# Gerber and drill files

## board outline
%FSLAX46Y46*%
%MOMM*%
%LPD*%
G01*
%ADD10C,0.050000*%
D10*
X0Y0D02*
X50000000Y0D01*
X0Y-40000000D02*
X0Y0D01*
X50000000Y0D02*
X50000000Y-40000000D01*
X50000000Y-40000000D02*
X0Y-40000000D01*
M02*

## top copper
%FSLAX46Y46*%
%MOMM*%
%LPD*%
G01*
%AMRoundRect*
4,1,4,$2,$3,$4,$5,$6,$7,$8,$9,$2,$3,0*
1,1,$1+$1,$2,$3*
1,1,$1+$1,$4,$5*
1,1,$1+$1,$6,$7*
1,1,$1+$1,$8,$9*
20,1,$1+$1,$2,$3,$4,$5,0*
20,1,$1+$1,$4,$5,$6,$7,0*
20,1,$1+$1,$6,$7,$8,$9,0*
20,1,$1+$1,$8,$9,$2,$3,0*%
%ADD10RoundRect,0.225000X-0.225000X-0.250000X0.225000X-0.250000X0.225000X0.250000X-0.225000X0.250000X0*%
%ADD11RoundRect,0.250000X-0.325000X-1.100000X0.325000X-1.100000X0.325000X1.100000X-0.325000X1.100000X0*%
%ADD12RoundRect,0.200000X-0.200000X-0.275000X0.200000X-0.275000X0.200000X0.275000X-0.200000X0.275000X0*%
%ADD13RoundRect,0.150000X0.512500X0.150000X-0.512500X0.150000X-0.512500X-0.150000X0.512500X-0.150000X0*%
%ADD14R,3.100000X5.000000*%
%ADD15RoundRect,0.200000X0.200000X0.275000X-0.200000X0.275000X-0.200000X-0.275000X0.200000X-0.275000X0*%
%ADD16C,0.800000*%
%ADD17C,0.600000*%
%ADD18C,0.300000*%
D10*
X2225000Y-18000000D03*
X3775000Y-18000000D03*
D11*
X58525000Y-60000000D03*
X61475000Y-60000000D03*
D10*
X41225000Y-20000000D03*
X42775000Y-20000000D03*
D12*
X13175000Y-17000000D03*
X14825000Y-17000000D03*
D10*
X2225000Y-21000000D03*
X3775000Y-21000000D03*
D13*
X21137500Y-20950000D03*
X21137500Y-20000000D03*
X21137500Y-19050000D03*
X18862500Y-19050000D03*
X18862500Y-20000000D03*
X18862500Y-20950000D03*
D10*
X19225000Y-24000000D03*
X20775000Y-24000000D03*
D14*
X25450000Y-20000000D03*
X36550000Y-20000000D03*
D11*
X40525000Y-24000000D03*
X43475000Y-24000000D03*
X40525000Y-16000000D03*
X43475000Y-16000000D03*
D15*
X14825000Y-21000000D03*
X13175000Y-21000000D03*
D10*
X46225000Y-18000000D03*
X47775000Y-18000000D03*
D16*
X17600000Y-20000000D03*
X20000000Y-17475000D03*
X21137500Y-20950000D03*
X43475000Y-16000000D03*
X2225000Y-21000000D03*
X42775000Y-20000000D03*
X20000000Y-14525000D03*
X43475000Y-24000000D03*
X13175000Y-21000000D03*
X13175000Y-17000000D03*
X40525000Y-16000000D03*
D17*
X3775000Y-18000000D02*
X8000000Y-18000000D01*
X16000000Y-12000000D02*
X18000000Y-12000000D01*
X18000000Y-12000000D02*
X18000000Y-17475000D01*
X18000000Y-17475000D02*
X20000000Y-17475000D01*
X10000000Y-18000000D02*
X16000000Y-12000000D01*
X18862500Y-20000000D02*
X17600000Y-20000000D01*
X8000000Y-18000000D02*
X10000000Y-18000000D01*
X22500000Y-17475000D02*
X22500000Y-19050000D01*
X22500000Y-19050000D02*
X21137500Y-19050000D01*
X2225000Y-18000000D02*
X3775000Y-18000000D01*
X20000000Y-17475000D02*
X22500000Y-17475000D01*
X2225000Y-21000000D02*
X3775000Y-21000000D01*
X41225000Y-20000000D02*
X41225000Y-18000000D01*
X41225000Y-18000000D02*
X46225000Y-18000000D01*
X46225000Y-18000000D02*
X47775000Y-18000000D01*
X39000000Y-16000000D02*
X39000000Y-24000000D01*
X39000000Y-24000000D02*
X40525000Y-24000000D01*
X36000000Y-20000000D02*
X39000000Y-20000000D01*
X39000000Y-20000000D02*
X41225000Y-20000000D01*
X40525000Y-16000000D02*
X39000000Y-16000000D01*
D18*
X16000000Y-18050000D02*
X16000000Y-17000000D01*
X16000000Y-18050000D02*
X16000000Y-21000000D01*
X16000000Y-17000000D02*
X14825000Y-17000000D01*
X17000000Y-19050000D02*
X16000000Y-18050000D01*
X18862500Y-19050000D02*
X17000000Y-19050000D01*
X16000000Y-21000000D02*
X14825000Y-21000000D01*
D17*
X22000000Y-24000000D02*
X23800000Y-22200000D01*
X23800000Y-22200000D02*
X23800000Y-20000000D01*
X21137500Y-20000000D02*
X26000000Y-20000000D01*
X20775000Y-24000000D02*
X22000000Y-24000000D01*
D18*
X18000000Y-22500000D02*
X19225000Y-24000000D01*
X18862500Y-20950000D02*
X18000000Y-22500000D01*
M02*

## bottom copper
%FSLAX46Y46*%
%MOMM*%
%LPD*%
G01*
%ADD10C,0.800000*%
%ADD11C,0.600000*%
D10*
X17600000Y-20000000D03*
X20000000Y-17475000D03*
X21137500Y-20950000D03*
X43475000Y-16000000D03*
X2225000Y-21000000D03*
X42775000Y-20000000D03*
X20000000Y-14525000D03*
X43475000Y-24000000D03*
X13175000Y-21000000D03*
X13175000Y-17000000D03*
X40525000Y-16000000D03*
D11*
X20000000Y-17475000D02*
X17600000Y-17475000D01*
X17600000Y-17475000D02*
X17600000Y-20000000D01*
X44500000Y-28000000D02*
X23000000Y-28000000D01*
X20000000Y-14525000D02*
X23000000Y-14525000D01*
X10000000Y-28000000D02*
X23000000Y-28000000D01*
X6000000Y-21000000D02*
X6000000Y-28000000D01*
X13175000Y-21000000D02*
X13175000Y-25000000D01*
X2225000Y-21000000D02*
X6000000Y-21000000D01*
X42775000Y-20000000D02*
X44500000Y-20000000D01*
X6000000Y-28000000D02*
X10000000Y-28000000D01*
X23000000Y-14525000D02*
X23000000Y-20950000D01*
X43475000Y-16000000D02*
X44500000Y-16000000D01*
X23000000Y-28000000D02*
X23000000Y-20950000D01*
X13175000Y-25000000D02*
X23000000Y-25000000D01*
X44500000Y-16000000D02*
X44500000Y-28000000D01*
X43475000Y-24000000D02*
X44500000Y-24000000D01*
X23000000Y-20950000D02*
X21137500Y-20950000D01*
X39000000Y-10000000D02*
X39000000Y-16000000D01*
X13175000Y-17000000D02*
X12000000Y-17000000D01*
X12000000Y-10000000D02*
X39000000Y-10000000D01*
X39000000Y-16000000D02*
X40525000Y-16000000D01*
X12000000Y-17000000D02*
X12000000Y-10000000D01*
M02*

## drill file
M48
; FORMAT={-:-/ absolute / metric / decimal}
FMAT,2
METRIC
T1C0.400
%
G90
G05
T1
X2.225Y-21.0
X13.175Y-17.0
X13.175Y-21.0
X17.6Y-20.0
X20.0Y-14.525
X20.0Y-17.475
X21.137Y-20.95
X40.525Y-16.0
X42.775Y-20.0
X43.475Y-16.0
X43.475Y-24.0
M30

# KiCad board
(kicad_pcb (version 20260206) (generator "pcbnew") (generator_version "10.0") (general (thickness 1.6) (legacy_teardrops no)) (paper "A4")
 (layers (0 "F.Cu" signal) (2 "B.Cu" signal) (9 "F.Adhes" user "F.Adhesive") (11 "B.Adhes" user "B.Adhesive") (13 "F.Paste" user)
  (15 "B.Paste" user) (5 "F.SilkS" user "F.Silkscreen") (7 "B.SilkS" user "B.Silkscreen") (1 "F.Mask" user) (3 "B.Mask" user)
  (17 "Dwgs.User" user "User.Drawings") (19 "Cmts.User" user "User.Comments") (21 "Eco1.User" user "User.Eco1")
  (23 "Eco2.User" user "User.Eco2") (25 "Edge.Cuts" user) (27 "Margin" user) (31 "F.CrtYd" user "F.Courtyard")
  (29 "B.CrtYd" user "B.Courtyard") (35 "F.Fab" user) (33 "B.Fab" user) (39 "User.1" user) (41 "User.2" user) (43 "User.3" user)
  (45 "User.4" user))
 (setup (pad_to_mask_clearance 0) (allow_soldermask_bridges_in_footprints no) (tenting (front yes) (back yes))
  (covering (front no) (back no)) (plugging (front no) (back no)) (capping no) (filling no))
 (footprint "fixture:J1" (layer "F.Cu") (at 3 18)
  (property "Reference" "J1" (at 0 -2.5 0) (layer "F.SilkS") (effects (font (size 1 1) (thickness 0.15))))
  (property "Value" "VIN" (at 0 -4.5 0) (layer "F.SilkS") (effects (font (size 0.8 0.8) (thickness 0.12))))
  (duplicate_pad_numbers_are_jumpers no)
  (pad "1" smd roundrect (at -0.775 0) (size 0.9 0.95) (layers "F.Cu" "F.Mask" "F.Paste") (roundrect_rratio 0.25) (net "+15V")
   (thermal_bridge_angle 45))
  (pad "2" smd roundrect (at 0.775 0) (size 0.9 0.95) (layers "F.Cu" "F.Mask" "F.Paste") (roundrect_rratio 0.25) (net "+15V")
   (thermal_bridge_angle 45)))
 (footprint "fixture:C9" (layer "F.Cu") (at 60 60)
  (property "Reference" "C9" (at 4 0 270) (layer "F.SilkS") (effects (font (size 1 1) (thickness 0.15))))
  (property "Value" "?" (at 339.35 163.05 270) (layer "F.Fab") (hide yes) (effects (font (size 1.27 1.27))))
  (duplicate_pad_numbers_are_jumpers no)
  (pad "1" smd roundrect (at -1.475 0) (size 1.15 2.7) (layers "F.Cu" "F.Mask" "F.Paste") (roundrect_rratio 0.217391) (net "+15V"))
  (pad "2" smd roundrect (at 1.475 0) (size 1.15 2.7) (layers "F.Cu" "F.Mask" "F.Paste") (roundrect_rratio 0.217391) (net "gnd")))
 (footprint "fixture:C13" (layer "F.Cu") (at 42 20)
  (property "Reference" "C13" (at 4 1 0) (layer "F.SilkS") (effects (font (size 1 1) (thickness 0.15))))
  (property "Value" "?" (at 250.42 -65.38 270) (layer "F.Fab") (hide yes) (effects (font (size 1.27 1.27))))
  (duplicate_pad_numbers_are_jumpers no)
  (pad "1" smd roundrect (at -0.775 0) (size 0.9 0.95) (layers "F.Cu" "F.Mask" "F.Paste") (roundrect_rratio 0.25) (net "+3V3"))
  (pad "2" smd roundrect (at 0.775 0) (size 0.9 0.95) (layers "F.Cu" "F.Mask" "F.Paste") (roundrect_rratio 0.25) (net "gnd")))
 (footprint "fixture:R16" (layer "F.Cu") (at 14 17)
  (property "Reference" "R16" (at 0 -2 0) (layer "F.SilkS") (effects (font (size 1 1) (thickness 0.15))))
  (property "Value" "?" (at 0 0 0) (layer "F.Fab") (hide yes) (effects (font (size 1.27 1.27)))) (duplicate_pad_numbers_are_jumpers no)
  (pad "1" smd roundrect (at -0.825 0) (size 0.8 0.95) (layers "F.Cu" "F.Mask" "F.Paste") (roundrect_rratio 0.25) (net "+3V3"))
  (pad "2" smd roundrect (at 0.825 0) (size 0.8 0.95) (layers "F.Cu" "F.Mask" "F.Paste") (roundrect_rratio 0.25) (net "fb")))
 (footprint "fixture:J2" (layer "F.Cu") (at 3 21)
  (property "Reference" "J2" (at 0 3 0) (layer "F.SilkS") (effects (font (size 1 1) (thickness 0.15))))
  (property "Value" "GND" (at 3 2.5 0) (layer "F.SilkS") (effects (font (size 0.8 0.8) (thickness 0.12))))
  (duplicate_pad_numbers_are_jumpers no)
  (pad "1" smd roundrect (at -0.775 0) (size 0.9 0.95) (layers "F.Cu" "F.Mask" "F.Paste") (roundrect_rratio 0.25) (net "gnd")
   (thermal_bridge_angle 45))
  (pad "2" smd roundrect (at 0.775 0) (size 0.9 0.95) (layers "F.Cu" "F.Mask" "F.Paste") (roundrect_rratio 0.25) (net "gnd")
   (thermal_bridge_angle 45)))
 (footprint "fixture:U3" (layer "F.Cu") (at 20 20 180)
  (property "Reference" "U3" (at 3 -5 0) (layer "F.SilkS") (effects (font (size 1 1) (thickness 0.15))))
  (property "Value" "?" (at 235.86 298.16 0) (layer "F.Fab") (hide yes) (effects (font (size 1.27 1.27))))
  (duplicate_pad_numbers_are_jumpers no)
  (pad "1" smd roundrect (at -1.1375 -0.95 180) (size 1.325 0.6) (layers "F.Cu" "F.Mask" "F.Paste") (roundrect_rratio 0.25) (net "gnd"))
  (pad "2" smd roundrect (at -1.1375 0 180) (size 1.325 0.6) (layers "F.Cu" "F.Mask" "F.Paste") (roundrect_rratio 0.25) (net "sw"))
  (pad "3" smd roundrect (at -1.1375 0.95 180) (size 1.325 0.6) (layers "F.Cu" "F.Mask" "F.Paste") (roundrect_rratio 0.25) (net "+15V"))
  (pad "4" smd roundrect (at 1.1375 0.95 180) (size 1.325 0.6) (layers "F.Cu" "F.Mask" "F.Paste") (roundrect_rratio 0.25) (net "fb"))
  (pad "5" smd roundrect (at 1.1375 0 180) (size 1.325 0.6) (layers "F.Cu" "F.Mask" "F.Paste") (roundrect_rratio 0.25) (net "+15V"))
  (pad "6" smd roundrect (at 1.1375 -0.95 180) (size 1.325 0.6) (layers "F.Cu" "F.Mask" "F.Paste") (roundrect_rratio 0.25) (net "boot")))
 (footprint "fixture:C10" (layer "F.Cu") (at 20 24)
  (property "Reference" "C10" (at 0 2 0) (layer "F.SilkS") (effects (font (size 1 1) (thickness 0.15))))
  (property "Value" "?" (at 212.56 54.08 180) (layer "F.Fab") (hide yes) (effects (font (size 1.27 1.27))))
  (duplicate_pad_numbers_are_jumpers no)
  (pad "1" smd roundrect (at -0.775 0) (size 0.9 0.95) (layers "F.Cu" "F.Mask" "F.Paste") (roundrect_rratio 0.25) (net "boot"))
  (pad "2" smd roundrect (at 0.775 0) (size 0.9 0.95) (layers "F.Cu" "F.Mask" "F.Paste") (roundrect_rratio 0.25) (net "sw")))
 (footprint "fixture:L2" (layer "F.Cu") (at 31 20)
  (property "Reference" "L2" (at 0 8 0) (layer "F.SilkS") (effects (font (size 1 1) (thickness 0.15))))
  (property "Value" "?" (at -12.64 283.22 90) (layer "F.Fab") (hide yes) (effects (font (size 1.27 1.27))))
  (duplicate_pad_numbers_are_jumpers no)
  (pad "1" smd rect (at -5.55 0) (size 3.1 5) (layers "F.Cu" "F.Mask" "F.Paste") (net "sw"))
  (pad "2" smd rect (at 5.55 0) (size 3.1 5) (layers "F.Cu" "F.Mask" "F.Paste") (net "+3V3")))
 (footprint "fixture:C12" (layer "F.Cu") (at 42 24)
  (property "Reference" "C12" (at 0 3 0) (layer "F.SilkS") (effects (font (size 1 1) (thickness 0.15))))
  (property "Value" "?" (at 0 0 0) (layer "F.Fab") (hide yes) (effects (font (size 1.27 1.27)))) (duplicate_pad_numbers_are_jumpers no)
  (pad "1" smd roundrect (at -1.475 0) (size 1.15 2.7) (layers "F.Cu" "F.Mask" "F.Paste") (roundrect_rratio 0.217391) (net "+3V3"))
  (pad "2" smd roundrect (at 1.475 0) (size 1.15 2.7) (layers "F.Cu" "F.Mask" "F.Paste") (roundrect_rratio 0.217391) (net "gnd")))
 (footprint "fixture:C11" (layer "F.Cu") (at 42 16)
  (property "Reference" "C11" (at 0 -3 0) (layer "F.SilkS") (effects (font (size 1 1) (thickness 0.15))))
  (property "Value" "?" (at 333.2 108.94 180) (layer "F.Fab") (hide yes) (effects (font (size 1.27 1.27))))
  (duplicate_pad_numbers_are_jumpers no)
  (pad "1" smd roundrect (at -1.475 0) (size 1.15 2.7) (layers "F.Cu" "F.Mask" "F.Paste") (roundrect_rratio 0.217391) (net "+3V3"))
  (pad "2" smd roundrect (at 1.475 0) (size 1.15 2.7) (layers "F.Cu" "F.Mask" "F.Paste") (roundrect_rratio 0.217391) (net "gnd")))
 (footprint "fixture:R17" (layer "F.Cu") (at 14 21 180)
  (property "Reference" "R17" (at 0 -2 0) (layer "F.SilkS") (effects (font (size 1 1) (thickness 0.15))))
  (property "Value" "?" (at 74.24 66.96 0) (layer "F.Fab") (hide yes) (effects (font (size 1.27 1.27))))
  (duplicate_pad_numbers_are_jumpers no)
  (pad "1" smd roundrect (at -0.825 0 180) (size 0.8 0.95) (layers "F.Cu" "F.Mask" "F.Paste") (roundrect_rratio 0.25) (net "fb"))
  (pad "2" smd roundrect (at 0.825 0 180) (size 0.8 0.95) (layers "F.Cu" "F.Mask" "F.Paste") (roundrect_rratio 0.25) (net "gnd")))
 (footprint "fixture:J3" (layer "F.Cu") (at 47 18)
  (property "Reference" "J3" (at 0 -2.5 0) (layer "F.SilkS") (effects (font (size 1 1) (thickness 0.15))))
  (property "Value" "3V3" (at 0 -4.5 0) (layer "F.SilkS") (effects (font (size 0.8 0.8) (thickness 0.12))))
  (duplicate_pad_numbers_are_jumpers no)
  (pad "1" smd roundrect (at -0.775 0) (size 0.9 0.95) (layers "F.Cu" "F.Mask" "F.Paste") (roundrect_rratio 0.25) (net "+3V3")
   (thermal_bridge_angle 45))
  (pad "2" smd roundrect (at 0.775 0) (size 0.9 0.95) (layers "F.Cu" "F.Mask" "F.Paste") (roundrect_rratio 0.25) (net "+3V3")
   (thermal_bridge_angle 45)))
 (gr_line (start 0 0) (end 50 0) (stroke (width 0.05) (type default)) (layer "Edge.Cuts"))
 (gr_line (start 0 40) (end 0 0) (stroke (width 0.05) (type default)) (layer "Edge.Cuts"))
 (gr_line (start 50 0) (end 50 40) (stroke (width 0.05) (type default)) (layer "Edge.Cuts"))
 (gr_line (start 50 40) (end 0 40) (stroke (width 0.05) (type default)) (layer "Edge.Cuts"))
 (segment (start 3.775 18) (end 8 18) (width 0.6) (layer "F.Cu") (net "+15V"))
 (segment (start 16 12) (end 18 12) (width 0.6) (layer "F.Cu") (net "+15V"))
 (segment (start 18 12) (end 18 17.475) (width 0.6) (layer "F.Cu") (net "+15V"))
 (segment (start 18 17.475) (end 20 17.475) (width 0.6) (layer "F.Cu") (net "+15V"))
 (segment (start 10 18) (end 16 12) (width 0.6) (layer "F.Cu") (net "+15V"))
 (segment (start 18.8625 20) (end 17.6 20) (width 0.6) (layer "F.Cu") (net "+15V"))
 (segment (start 8 18) (end 10 18) (width 0.6) (layer "F.Cu") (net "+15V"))
 (segment (start 22.5 17.475) (end 22.5 19.05) (width 0.6) (layer "F.Cu") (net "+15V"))
 (segment (start 22.5 19.05) (end 21.1375 19.05) (width 0.6) (layer "F.Cu") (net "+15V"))
 (segment (start 2.225 18) (end 3.775 18) (width 0.6) (layer "F.Cu") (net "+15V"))
 (segment (start 20 17.475) (end 22.5 17.475) (width 0.6) (layer "F.Cu") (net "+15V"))
 (via (at 17.6 20) (size 0.8) (drill 0.4) (layers "F.Cu" "B.Cu") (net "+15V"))
 (via (at 20 17.475) (size 0.8) (drill 0.4) (layers "F.Cu" "B.Cu") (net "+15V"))
 (segment (start 20 17.475) (end 17.6 17.475) (width 0.6) (layer "B.Cu") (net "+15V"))
 (segment (start 17.6 17.475) (end 17.6 20) (width 0.6) (layer "B.Cu") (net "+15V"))
 (segment (start 2.225 21) (end 3.775 21) (width 0.6) (layer "F.Cu") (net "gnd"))
 (via (at 21.1375 20.95) (size 0.8) (drill 0.4) (layers "F.Cu" "B.Cu") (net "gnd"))
 (via (at 43.475 16) (size 0.8) (drill 0.4) (layers "F.Cu" "B.Cu") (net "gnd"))
 (via (at 2.225 21) (size 0.8) (drill 0.4) (layers "F.Cu" "B.Cu") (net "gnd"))
 (via (at 42.775 20) (size 0.8) (drill 0.4) (layers "F.Cu" "B.Cu") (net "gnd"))
 (via (at 20 14.525) (size 0.8) (drill 0.4) (layers "F.Cu" "B.Cu") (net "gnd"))
 (via (at 43.475 24) (size 0.8) (drill 0.4) (layers "F.Cu" "B.Cu") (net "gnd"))
 (via (at 13.175 21) (size 0.8) (drill 0.4) (layers "F.Cu" "B.Cu") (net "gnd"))
 (segment (start 44.5 28) (end 23 28) (width 0.6) (layer "B.Cu") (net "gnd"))
 (segment (start 20 14.525) (end 23 14.525) (width 0.6) (layer "B.Cu") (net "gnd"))
 (segment (start 10 28) (end 23 28) (width 0.6) (layer "B.Cu") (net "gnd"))
 (segment (start 6 21) (end 6 28) (width 0.6) (layer "B.Cu") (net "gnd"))
 (segment (start 13.175 21) (end 13.175 25) (width 0.6) (layer "B.Cu") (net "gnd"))
 (segment (start 2.225 21) (end 6 21) (width 0.6) (layer "B.Cu") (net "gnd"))
 (segment (start 42.775 20) (end 44.5 20) (width 0.6) (layer "B.Cu") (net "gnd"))
 (segment (start 6 28) (end 10 28) (width 0.6) (layer "B.Cu") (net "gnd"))
 (segment (start 23 14.525) (end 23 20.95) (width 0.6) (layer "B.Cu") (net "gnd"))
 (segment (start 43.475 16) (end 44.5 16) (width 0.6) (layer "B.Cu") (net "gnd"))
 (segment (start 23 28) (end 23 20.95) (width 0.6) (layer "B.Cu") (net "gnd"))
 (segment (start 13.175 25) (end 23 25) (width 0.6) (layer "B.Cu") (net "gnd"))
 (segment (start 44.5 16) (end 44.5 28) (width 0.6) (layer "B.Cu") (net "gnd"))
 (segment (start 43.475 24) (end 44.5 24) (width 0.6) (layer "B.Cu") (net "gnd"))
 (segment (start 23 20.95) (end 21.1375 20.95) (width 0.6) (layer "B.Cu") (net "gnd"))
 (segment (start 41.225 20) (end 41.225 18) (width 0.6) (layer "F.Cu") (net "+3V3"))
 (segment (start 41.225 18) (end 46.225 18) (width 0.6) (layer "F.Cu") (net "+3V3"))
 (segment (start 46.225 18) (end 47.775 18) (width 0.6) (layer "F.Cu") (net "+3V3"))
 (segment (start 39 16) (end 39 24) (width 0.6) (layer "F.Cu") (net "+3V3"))
 (segment (start 39 24) (end 40.525 24) (width 0.6) (layer "F.Cu") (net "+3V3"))
 (segment (start 36 20) (end 39 20) (width 0.6) (layer "F.Cu") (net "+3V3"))
 (segment (start 39 20) (end 41.225 20) (width 0.6) (layer "F.Cu") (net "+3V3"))
 (segment (start 40.525 16) (end 39 16) (width 0.6) (layer "F.Cu") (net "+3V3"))
 (via (at 13.175 17) (size 0.8) (drill 0.4) (layers "F.Cu" "B.Cu") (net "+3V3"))
 (via (at 40.525 16) (size 0.8) (drill 0.4) (layers "F.Cu" "B.Cu") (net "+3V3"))
 (segment (start 39 10) (end 39 16) (width 0.6) (layer "B.Cu") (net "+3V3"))
 (segment (start 13.175 17) (end 12 17) (width 0.6) (layer "B.Cu") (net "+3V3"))
 (segment (start 12 10) (end 39 10) (width 0.6) (layer "B.Cu") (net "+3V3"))
 (segment (start 39 16) (end 40.525 16) (width 0.6) (layer "B.Cu") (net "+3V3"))
 (segment (start 12 17) (end 12 10) (width 0.6) (layer "B.Cu") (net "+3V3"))
 (segment (start 16 18.05) (end 16 17) (width 0.3) (layer "F.Cu") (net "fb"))
 (segment (start 16 18.05) (end 16 21) (width 0.3) (layer "F.Cu") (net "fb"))
 (segment (start 16 17) (end 14.825 17) (width 0.3) (layer "F.Cu") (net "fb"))
 (segment (start 17 19.05) (end 16 18.05) (width 0.3) (layer "F.Cu") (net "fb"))
 (segment (start 18.8625 19.05) (end 17 19.05) (width 0.3) (layer "F.Cu") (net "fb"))
 (segment (start 16 21) (end 14.825 21) (width 0.3) (layer "F.Cu") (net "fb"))
 (segment (start 22 24) (end 23.8 22.2) (width 0.6) (layer "F.Cu") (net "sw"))
 (segment (start 23.8 22.2) (end 23.8 20) (width 0.6) (layer "F.Cu") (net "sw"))
 (segment (start 21.1375 20) (end 26 20) (width 0.6) (layer "F.Cu") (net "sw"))
 (segment (start 20.775 24) (end 22 24) (width 0.6) (layer "F.Cu") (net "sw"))
 (segment (start 18 22.5) (end 19.225 24) (width 0.3) (layer "F.Cu") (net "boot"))
 (segment (start 18.8625 20.95) (end 18 22.5) (width 0.3) (layer "F.Cu") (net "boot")))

